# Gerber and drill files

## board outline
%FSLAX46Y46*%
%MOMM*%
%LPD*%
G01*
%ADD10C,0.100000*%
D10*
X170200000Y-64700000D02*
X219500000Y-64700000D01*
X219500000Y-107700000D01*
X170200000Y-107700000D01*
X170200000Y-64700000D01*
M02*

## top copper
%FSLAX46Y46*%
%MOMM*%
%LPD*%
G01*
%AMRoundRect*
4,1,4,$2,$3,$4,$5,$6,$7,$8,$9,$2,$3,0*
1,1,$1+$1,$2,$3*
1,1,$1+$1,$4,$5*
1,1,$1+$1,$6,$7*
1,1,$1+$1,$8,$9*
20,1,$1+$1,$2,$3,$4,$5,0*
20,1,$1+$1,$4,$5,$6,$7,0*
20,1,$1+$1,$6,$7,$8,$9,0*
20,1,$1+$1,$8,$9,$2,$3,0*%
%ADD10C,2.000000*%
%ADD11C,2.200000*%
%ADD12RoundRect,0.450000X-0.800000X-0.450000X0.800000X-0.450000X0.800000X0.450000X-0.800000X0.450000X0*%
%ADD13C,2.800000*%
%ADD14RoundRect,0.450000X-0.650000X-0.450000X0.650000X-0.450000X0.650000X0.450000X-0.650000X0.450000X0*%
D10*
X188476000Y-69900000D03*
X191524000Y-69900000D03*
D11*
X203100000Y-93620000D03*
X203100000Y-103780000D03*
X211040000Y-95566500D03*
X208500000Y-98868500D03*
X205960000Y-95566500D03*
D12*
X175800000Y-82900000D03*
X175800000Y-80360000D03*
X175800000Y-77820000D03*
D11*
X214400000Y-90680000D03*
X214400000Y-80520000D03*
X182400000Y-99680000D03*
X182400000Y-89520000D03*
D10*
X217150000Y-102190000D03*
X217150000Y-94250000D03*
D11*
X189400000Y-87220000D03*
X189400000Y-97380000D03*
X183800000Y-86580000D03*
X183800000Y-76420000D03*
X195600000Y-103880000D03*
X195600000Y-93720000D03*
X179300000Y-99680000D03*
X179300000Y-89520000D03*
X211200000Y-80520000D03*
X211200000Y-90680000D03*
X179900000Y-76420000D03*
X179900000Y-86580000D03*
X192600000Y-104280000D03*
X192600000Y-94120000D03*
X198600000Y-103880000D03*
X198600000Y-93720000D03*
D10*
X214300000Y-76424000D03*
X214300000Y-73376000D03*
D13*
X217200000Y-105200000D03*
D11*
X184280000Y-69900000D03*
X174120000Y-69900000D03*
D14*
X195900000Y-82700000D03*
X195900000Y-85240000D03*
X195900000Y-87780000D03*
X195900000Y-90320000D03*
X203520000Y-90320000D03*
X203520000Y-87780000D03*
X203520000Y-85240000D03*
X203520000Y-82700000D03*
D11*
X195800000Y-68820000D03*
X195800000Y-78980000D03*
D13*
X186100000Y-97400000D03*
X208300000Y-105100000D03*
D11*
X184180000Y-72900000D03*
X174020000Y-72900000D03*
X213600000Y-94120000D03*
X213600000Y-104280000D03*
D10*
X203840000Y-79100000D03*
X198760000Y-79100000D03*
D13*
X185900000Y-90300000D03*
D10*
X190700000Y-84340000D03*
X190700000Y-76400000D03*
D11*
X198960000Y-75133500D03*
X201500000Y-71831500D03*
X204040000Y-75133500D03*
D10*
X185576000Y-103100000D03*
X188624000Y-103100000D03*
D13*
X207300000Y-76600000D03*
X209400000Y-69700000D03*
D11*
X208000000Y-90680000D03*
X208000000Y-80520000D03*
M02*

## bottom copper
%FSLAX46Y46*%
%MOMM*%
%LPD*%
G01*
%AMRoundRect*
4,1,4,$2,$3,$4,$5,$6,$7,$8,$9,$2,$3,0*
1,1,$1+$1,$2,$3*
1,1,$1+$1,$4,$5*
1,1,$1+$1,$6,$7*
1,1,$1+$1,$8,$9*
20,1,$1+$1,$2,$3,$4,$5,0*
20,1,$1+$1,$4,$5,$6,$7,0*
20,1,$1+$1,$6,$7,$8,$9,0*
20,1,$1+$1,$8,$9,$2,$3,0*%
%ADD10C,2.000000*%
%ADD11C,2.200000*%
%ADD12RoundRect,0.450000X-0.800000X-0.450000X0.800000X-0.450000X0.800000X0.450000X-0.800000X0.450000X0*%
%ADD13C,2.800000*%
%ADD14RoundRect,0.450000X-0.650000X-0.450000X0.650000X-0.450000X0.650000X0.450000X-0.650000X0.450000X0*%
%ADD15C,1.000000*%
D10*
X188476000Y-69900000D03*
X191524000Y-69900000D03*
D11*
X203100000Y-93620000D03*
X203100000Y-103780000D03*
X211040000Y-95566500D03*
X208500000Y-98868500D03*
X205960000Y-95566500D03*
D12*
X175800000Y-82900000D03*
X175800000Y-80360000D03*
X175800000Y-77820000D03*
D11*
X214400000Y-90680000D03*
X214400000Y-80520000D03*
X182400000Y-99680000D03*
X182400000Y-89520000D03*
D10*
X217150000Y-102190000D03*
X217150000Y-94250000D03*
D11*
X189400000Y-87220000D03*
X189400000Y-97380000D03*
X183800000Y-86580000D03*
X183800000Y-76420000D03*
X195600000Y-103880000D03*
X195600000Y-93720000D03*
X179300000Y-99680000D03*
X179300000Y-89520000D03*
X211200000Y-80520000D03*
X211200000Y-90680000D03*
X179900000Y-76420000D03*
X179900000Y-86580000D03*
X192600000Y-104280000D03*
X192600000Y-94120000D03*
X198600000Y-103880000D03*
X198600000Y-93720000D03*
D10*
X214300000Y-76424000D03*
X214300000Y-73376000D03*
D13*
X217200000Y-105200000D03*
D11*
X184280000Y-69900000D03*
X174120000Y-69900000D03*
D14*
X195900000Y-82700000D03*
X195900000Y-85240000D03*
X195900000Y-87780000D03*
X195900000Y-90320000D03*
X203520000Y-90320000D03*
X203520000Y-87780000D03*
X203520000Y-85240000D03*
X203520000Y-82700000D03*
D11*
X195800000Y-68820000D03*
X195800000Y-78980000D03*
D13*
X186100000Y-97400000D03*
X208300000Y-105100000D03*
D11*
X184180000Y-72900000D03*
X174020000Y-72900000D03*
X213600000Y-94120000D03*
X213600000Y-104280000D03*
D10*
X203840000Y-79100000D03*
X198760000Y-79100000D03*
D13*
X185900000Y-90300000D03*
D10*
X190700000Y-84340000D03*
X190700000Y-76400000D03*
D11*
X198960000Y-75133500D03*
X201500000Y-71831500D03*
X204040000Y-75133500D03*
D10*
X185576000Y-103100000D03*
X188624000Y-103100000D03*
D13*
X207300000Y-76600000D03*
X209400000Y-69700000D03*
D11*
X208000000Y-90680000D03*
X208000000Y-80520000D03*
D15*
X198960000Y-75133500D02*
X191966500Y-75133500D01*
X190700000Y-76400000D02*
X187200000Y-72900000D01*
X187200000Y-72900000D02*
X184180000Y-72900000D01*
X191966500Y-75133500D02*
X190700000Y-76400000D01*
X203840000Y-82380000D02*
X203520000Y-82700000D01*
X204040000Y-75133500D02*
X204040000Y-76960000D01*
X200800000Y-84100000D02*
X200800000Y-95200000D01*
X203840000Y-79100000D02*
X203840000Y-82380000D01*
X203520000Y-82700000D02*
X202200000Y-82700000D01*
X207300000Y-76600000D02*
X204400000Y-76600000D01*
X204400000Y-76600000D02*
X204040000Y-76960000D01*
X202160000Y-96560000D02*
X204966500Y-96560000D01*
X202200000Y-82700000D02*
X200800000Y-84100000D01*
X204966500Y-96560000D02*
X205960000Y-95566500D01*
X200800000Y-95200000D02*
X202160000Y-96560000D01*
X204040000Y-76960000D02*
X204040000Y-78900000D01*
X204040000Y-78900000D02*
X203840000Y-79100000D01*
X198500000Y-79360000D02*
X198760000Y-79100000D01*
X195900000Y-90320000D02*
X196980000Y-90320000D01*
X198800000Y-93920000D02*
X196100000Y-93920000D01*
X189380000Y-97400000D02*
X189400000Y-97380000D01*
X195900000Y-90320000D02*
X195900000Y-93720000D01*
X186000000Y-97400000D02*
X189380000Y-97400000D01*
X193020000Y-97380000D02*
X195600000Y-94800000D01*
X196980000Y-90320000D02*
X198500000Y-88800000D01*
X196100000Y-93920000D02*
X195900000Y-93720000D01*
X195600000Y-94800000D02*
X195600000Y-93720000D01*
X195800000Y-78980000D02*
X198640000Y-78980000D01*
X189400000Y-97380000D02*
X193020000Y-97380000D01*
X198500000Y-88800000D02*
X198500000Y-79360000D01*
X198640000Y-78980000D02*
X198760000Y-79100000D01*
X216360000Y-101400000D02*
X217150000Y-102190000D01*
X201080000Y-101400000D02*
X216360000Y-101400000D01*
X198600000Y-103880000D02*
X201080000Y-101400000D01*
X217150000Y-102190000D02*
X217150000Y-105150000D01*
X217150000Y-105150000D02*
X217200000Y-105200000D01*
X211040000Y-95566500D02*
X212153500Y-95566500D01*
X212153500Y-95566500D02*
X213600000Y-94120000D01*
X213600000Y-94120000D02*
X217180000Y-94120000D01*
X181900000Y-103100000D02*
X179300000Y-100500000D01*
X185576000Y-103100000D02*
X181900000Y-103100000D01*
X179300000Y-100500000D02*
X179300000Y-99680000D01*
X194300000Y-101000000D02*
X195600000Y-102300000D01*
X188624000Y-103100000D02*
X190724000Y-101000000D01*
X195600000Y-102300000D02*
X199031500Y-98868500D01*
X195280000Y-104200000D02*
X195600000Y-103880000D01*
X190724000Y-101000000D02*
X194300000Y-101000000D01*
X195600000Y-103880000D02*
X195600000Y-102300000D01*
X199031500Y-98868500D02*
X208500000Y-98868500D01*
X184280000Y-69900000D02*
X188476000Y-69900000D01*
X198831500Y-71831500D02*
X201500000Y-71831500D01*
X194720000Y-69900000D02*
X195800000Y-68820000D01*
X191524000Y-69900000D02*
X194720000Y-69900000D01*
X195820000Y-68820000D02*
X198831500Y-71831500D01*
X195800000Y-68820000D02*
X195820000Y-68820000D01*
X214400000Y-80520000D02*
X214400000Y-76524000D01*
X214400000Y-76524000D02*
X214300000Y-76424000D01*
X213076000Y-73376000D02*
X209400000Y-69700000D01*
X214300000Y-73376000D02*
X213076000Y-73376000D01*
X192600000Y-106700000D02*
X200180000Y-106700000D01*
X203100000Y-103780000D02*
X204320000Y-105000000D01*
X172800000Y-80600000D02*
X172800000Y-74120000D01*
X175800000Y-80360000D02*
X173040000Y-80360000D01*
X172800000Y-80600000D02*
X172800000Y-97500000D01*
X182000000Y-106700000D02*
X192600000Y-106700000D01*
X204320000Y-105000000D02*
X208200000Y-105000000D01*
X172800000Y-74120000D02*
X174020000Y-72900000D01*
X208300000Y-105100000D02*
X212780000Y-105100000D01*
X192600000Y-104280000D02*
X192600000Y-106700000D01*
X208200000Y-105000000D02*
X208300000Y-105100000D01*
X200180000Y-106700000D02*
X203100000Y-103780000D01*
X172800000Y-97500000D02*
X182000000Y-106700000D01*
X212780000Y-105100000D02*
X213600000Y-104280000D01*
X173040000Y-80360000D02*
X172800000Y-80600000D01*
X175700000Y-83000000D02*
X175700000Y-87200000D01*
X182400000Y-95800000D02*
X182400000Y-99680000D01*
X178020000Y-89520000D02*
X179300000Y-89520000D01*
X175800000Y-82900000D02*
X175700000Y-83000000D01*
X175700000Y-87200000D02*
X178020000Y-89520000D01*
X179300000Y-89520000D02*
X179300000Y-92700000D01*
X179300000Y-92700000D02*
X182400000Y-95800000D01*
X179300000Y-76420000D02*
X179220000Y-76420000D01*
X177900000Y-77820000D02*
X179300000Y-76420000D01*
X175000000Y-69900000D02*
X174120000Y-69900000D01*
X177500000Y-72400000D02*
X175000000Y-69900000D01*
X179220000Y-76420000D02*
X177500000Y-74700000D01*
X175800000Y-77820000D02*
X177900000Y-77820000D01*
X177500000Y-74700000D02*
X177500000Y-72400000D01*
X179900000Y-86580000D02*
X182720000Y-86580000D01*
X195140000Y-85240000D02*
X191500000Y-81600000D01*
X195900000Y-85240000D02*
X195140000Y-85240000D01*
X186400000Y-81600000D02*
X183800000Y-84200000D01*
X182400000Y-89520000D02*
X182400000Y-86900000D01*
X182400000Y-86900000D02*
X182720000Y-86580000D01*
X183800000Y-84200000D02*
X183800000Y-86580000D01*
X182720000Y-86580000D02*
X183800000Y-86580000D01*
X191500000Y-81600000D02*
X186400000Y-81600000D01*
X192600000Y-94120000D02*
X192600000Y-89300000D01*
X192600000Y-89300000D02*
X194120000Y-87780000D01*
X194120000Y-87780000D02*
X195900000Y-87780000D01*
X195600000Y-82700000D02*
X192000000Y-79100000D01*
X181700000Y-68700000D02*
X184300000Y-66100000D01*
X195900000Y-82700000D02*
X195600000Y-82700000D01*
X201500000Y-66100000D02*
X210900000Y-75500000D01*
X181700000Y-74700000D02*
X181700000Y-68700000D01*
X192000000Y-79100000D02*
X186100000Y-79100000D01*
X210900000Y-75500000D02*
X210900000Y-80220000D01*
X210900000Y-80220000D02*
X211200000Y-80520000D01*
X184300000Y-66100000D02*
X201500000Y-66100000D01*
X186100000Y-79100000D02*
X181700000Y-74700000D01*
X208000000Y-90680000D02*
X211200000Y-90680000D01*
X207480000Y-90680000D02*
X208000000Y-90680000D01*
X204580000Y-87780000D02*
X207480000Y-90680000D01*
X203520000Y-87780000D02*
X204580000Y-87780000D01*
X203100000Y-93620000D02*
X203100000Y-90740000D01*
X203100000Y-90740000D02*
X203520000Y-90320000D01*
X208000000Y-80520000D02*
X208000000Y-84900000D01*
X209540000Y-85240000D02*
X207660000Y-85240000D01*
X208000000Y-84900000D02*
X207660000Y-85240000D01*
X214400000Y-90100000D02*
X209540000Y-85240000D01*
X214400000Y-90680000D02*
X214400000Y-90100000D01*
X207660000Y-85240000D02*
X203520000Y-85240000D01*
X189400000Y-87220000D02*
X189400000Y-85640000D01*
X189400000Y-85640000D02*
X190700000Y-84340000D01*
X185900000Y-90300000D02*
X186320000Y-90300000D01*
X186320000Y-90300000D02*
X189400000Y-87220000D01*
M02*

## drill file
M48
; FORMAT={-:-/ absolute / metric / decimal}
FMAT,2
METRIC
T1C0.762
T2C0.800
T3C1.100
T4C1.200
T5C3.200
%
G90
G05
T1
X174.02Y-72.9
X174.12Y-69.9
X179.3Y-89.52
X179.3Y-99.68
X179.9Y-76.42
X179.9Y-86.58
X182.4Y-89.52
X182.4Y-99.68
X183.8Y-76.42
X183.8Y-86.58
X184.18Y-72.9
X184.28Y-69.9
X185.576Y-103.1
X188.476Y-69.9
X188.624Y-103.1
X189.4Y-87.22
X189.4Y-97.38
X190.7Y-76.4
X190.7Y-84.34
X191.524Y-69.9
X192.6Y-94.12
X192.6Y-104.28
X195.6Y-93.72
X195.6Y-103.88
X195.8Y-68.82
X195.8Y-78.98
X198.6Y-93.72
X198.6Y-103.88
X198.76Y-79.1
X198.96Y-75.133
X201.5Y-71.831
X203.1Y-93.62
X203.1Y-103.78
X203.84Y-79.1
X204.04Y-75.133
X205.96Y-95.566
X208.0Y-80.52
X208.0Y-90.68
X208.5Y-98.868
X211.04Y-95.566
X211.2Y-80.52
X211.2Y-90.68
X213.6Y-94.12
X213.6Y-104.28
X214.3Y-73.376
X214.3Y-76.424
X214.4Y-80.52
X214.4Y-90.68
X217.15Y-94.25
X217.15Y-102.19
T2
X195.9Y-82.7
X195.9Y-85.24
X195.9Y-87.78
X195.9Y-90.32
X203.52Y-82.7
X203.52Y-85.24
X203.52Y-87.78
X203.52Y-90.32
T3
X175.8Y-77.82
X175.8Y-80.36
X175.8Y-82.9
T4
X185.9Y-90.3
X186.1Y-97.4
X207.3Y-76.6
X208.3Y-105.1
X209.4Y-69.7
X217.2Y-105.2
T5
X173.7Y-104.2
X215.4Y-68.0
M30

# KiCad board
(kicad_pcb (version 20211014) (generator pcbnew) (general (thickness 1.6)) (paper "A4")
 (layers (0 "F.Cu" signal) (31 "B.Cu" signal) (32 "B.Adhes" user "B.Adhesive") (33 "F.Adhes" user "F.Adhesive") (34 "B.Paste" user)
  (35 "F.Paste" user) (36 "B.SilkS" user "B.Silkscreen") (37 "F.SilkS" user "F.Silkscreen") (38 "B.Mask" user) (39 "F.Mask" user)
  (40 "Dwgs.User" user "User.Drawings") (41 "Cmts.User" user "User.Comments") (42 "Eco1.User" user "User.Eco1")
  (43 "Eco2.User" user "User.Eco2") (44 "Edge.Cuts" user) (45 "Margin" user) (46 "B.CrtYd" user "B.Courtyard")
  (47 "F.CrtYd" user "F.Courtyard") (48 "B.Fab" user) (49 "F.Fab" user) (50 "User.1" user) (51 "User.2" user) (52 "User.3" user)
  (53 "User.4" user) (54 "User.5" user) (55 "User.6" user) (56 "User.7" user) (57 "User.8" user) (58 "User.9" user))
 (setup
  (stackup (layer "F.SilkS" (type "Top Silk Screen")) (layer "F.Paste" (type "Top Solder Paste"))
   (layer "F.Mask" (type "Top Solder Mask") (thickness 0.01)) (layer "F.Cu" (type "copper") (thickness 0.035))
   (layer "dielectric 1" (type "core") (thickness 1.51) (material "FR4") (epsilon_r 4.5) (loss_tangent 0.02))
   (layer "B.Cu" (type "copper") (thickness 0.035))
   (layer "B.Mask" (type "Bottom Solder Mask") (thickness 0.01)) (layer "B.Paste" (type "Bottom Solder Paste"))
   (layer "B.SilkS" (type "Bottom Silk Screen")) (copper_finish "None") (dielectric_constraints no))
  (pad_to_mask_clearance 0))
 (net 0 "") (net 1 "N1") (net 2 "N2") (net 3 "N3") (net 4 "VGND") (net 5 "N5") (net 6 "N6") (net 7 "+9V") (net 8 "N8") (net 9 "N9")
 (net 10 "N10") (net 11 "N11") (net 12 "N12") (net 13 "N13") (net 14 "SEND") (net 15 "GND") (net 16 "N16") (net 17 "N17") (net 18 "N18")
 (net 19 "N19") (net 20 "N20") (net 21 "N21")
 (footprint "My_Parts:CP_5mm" (layer "F.Cu") (at 190 69.9)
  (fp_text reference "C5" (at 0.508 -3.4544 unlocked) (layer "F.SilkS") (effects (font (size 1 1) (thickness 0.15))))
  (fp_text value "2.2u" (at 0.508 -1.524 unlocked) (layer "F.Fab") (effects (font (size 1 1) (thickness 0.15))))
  (pad "1" thru_hole circle (at -1.524 0) (size 2 2) (drill 0.762) (layers *.Cu *.Mask) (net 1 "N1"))
  (pad "2" thru_hole circle (at 1.524 0) (size 2 2) (drill 0.762) (layers *.Cu *.Mask) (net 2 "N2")))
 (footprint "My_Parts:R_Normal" (layer "F.Cu") (at 203.1 98.7 -90)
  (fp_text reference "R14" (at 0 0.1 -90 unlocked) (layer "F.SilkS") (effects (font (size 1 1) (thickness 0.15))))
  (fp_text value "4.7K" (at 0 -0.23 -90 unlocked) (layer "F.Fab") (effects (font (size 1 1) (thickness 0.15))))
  (pad "1" thru_hole circle (at -5.08 0 270) (size 2.2 2.2) (drill 0.762) (layers *.Cu *.Mask) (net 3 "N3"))
  (pad "2" thru_hole circle (at 5.08 0 270) (size 2.2 2.2) (drill 0.762) (layers *.Cu *.Mask) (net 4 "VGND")))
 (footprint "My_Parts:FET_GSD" (layer "F.Cu") (at 211.04 96.5825 180)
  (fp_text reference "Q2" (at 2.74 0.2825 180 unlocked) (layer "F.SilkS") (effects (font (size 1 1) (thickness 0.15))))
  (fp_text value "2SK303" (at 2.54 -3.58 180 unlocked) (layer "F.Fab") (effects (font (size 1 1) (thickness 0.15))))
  (pad "1" thru_hole circle (at 0 1.016 180) (size 2.2 2.2) (drill 0.762) (layers *.Cu *.Mask) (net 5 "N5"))
  (pad "2" thru_hole circle (at 2.54 -2.286 180) (size 2.2 2.2) (drill 0.762) (layers *.Cu *.Mask) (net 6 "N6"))
  (pad "3" thru_hole circle (at 5.08 1.016 180) (size 2.2 2.2) (drill 0.762) (layers *.Cu *.Mask) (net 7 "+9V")))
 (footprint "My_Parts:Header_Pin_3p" (layer "F.Cu") (at 175.8 82.9)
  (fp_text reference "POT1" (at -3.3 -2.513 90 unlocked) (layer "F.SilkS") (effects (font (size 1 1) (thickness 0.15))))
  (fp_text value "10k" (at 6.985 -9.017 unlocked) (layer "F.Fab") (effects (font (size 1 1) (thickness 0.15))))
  (pad "1" thru_hole roundrect (at 0 0) (size 2.5 1.8) (drill 1.1) (layers *.Cu *.Mask) (roundrect_rratio 0.25) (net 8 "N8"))
  (pad "2" thru_hole roundrect (at 0 -2.54) (size 2.5 1.8) (drill 1.1) (layers *.Cu *.Mask) (roundrect_rratio 0.25) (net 4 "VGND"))
  (pad "3" thru_hole roundrect (at 0 -5.08) (size 2.5 1.8) (drill 1.1) (layers *.Cu *.Mask) (roundrect_rratio 0.25) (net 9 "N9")))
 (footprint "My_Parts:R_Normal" (layer "F.Cu") (at 214.4 85.6 90)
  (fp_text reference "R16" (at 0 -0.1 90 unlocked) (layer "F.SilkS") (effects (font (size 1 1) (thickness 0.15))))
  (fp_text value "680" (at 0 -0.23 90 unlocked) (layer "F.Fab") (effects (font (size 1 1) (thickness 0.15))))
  (pad "1" thru_hole circle (at -5.08 0 90) (size 2.2 2.2) (drill 0.762) (layers *.Cu *.Mask) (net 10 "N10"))
  (pad "2" thru_hole circle (at 5.08 0 90) (size 2.2 2.2) (drill 0.762) (layers *.Cu *.Mask) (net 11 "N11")))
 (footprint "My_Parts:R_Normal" (layer "F.Cu") (at 182.4 94.6 90)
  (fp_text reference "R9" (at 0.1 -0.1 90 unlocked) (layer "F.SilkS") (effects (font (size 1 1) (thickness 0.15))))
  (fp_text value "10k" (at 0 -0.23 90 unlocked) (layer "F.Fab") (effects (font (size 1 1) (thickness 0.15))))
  (pad "1" thru_hole circle (at -5.08 0 90) (size 2.2 2.2) (drill 0.762) (layers *.Cu *.Mask) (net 8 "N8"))
  (pad "2" thru_hole circle (at 5.08 0 90) (size 2.2 2.2) (drill 0.762) (layers *.Cu *.Mask) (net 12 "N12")))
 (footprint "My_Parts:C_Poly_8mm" (layer "F.Cu") (at 217.15 99.65 90)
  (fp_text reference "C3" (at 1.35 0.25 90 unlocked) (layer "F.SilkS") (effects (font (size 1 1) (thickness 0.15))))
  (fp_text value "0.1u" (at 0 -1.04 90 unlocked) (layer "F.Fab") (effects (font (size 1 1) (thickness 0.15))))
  (pad "1" thru_hole circle (at -2.54 0 90) (size 2 2) (drill 0.762) (layers *.Cu *.Mask) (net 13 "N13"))
  (pad "2" thru_hole circle (at 5.4 0 90) (size 2 2) (drill 0.762) (layers *.Cu *.Mask) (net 5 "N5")))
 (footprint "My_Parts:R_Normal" (layer "F.Cu") (at 189.4 92.3 -90)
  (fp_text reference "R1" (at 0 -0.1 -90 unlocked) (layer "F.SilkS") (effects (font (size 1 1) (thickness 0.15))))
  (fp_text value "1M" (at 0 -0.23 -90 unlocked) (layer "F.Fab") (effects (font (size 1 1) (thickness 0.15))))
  (pad "1" thru_hole circle (at -5.08 0 270) (size 2.2 2.2) (drill 0.762) (layers *.Cu *.Mask) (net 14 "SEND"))
  (pad "2" thru_hole circle (at 5.08 0 270) (size 2.2 2.2) (drill 0.762) (layers *.Cu *.Mask) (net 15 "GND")))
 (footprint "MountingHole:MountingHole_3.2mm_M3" (layer "F.Cu") (at 173.7 104.2)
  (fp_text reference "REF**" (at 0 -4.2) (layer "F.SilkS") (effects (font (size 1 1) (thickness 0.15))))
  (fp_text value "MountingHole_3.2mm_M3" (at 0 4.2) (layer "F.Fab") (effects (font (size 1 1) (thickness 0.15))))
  (pad "" np_thru_hole circle (at 0 0) (size 3.2 3.2) (drill 3.2) (layers F&B.Cu *.Mask)))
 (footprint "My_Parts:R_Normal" (layer "F.Cu") (at 183.8 81.5 90)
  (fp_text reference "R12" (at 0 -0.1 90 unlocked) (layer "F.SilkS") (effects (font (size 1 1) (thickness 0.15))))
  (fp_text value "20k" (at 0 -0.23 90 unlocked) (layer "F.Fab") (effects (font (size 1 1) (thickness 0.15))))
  (pad "1" thru_hole circle (at -5.08 0 90) (size 2.2 2.2) (drill 0.762) (layers *.Cu *.Mask) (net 12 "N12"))
  (pad "2" thru_hole circle (at 5.08 0 90) (size 2.2 2.2) (drill 0.762) (layers *.Cu *.Mask) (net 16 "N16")))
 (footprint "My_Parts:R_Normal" (layer "F.Cu") (at 195.6 98.8 90)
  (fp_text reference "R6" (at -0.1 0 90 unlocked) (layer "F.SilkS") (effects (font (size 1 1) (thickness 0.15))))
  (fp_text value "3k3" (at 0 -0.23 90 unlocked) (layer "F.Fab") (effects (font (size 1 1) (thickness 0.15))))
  (pad "1" thru_hole circle (at -5.08 0 90) (size 2.2 2.2) (drill 0.762) (layers *.Cu *.Mask) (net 6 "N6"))
  (pad "2" thru_hole circle (at 5.08 0 90) (size 2.2 2.2) (drill 0.762) (layers *.Cu *.Mask) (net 15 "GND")))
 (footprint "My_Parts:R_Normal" (layer "F.Cu") (at 179.3 94.6 90)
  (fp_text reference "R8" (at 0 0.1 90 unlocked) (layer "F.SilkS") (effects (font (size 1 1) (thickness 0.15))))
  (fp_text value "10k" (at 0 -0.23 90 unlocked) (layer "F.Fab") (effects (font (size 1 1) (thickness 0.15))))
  (pad "1" thru_hole circle (at -5.08 0 90) (size 2.2 2.2) (drill 0.762) (layers *.Cu *.Mask) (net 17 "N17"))
  (pad "2" thru_hole circle (at 5.08 0 90) (size 2.2 2.2) (drill 0.762) (layers *.Cu *.Mask) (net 8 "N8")))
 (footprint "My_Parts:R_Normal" (layer "F.Cu") (at 211.2 85.6 -90)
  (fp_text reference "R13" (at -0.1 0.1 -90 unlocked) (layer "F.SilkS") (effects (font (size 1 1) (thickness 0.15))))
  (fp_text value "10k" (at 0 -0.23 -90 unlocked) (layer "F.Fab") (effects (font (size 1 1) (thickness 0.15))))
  (pad "1" thru_hole circle (at -5.08 0 270) (size 2.2 2.2) (drill 0.762) (layers *.Cu *.Mask) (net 16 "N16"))
  (pad "2" thru_hole circle (at 5.08 0 270) (size 2.2 2.2) (drill 0.762) (layers *.Cu *.Mask) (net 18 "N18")))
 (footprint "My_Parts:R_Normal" (layer "F.Cu") (at 179.9 81.5 -90)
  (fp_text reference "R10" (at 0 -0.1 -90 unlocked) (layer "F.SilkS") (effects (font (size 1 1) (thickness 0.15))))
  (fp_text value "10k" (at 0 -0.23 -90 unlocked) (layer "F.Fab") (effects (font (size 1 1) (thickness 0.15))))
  (pad "1" thru_hole circle (at -5.08 0 270) (size 2.2 2.2) (drill 0.762) (layers *.Cu *.Mask) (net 9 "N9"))
  (pad "2" thru_hole circle (at 5.08 0 270) (size 2.2 2.2) (drill 0.762) (layers *.Cu *.Mask) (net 12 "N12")))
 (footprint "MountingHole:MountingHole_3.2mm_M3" (layer "F.Cu") (at 215.4 68)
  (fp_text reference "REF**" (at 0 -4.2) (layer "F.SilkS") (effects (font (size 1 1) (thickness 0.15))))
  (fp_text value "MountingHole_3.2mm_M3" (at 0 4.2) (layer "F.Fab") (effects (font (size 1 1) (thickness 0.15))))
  (pad "" np_thru_hole circle (at 0 0) (size 3.2 3.2) (drill 3.2) (layers *.Cu *.Mask)))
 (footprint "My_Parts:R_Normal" (layer "F.Cu") (at 192.6 99.2 90)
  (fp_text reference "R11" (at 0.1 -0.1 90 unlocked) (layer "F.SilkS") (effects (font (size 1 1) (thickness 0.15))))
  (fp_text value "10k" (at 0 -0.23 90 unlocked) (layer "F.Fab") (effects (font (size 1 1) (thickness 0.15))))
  (pad "1" thru_hole circle (at -5.08 0 90) (size 2.2 2.2) (drill 0.762) (layers *.Cu *.Mask) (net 4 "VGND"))
  (pad "2" thru_hole circle (at 5.08 0 90) (size 2.2 2.2) (drill 0.762) (layers *.Cu *.Mask) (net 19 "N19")))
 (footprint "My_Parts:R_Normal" (layer "F.Cu") (at 198.6 98.8 90)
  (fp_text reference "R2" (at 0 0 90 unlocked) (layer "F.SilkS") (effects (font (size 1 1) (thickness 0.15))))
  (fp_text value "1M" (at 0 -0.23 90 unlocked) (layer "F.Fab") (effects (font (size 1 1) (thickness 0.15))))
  (pad "1" thru_hole circle (at -5.08 0 90) (size 2.2 2.2) (drill 0.762) (layers *.Cu *.Mask) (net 13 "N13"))
  (pad "2" thru_hole circle (at 5.08 0 90) (size 2.2 2.2) (drill 0.762) (layers *.Cu *.Mask) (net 15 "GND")))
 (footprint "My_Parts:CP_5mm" (layer "F.Cu") (at 214.3 74.9 90)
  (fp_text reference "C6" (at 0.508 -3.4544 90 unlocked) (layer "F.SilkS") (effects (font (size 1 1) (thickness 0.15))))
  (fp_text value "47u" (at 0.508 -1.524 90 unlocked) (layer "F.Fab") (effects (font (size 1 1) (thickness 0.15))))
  (pad "1" thru_hole circle (at -1.524 0 90) (size 2 2) (drill 0.762) (layers *.Cu *.Mask) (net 11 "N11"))
  (pad "2" thru_hole circle (at 1.524 0 90) (size 2 2) (drill 0.762) (layers *.Cu *.Mask) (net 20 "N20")))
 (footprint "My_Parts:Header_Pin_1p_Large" (layer "F.Cu") (at 217.2 105.2)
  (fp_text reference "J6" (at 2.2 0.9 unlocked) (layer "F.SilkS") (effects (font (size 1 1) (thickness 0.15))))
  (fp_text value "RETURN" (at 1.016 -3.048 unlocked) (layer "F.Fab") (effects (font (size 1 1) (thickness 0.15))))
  (pad "1" thru_hole circle (at 0 0) (size 2.8 2.8) (drill 1.2) (layers *.Cu *.Mask) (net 13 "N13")))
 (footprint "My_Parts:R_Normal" (layer "F.Cu") (at 179.2 69.9 180)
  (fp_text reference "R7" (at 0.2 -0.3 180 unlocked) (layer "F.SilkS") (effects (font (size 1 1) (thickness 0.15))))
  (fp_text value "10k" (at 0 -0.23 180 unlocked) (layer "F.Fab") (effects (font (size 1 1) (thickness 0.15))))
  (pad "1" thru_hole circle (at -5.08 0 180) (size 2.2 2.2) (drill 0.762) (layers *.Cu *.Mask) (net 1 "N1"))
  (pad "2" thru_hole circle (at 5.08 0 180) (size 2.2 2.2) (drill 0.762) (layers *.Cu *.Mask) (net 9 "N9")))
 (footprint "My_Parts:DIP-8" (layer "F.Cu") (at 197.17 83.2)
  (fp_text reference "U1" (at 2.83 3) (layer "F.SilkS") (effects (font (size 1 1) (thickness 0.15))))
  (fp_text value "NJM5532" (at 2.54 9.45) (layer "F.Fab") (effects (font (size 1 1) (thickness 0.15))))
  (pad "1" thru_hole roundrect (at -1.27 -0.5) (size 2.2 1.8) (drill 0.8) (layers *.Cu *.Mask) (roundrect_rratio 0.25) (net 16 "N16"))
  (pad "2" thru_hole roundrect (at -1.27 2.04) (size 2.2 1.8) (drill 0.8) (layers *.Cu *.Mask) (roundrect_rratio 0.25) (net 12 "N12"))
  (pad "3" thru_hole roundrect (at -1.27 4.58) (size 2.2 1.8) (drill 0.8) (layers *.Cu *.Mask) (roundrect_rratio 0.25) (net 19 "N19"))
  (pad "4" thru_hole roundrect (at -1.27 7.12) (size 2.2 1.8) (drill 0.8) (layers *.Cu *.Mask) (roundrect_rratio 0.25) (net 15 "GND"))
  (pad "5" thru_hole roundrect (at 6.35 7.12) (size 2.2 1.8) (drill 0.8) (layers *.Cu *.Mask) (roundrect_rratio 0.25) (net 3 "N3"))
  (pad "6" thru_hole roundrect (at 6.35 4.58) (size 2.2 1.8) (drill 0.8) (layers *.Cu *.Mask) (roundrect_rratio 0.25) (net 18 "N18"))
  (pad "7" thru_hole roundrect (at 6.35 2.04) (size 2.2 1.8) (drill 0.8) (layers *.Cu *.Mask) (roundrect_rratio 0.25) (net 10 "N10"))
  (pad "8" thru_hole roundrect (at 6.35 -0.5) (size 2.2 1.8) (drill 0.8) (layers *.Cu *.Mask) (roundrect_rratio 0.25) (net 7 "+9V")))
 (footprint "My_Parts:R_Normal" (layer "F.Cu") (at 195.8 73.9 -90)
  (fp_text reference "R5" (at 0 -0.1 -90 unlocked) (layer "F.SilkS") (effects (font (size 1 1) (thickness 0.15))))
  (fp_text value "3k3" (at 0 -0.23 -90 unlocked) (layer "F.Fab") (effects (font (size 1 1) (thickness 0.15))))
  (pad "1" thru_hole circle (at -5.08 0 270) (size 2.2 2.2) (drill 0.762) (layers *.Cu *.Mask) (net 2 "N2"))
  (pad "2" thru_hole circle (at 5.08 0 270) (size 2.2 2.2) (drill 0.762) (layers *.Cu *.Mask) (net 15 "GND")))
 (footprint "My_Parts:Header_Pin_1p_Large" (layer "F.Cu") (at 186.1 97.4)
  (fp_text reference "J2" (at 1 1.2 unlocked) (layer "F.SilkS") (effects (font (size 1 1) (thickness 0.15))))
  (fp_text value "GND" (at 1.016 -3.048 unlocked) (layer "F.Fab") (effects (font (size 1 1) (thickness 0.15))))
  (pad "1" thru_hole circle (at 0 0) (size 2.8 2.8) (drill 1.2) (layers *.Cu *.Mask) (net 15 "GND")))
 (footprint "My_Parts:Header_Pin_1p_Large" (layer "F.Cu") (at 208.3 105.1)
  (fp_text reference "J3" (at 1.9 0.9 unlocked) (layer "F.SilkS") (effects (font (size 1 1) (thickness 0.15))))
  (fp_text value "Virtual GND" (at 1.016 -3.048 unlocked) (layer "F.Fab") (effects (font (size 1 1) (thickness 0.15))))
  (pad "1" thru_hole circle (at 0 0) (size 2.8 2.8) (drill 1.2) (layers *.Cu *.Mask) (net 4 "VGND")))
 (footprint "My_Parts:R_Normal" (layer "F.Cu") (at 179.1 72.9 180)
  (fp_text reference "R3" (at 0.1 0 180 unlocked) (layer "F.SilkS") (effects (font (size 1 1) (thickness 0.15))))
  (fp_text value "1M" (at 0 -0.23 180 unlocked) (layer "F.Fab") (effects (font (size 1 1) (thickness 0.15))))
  (pad "1" thru_hole circle (at -5.08 0 180) (size 2.2 2.2) (drill 0.762) (layers *.Cu *.Mask) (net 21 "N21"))
  (pad "2" thru_hole circle (at 5.08 0 180) (size 2.2 2.2) (drill 0.762) (layers *.Cu *.Mask) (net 4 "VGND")))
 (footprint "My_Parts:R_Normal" (layer "F.Cu") (at 213.6 99.2 -90)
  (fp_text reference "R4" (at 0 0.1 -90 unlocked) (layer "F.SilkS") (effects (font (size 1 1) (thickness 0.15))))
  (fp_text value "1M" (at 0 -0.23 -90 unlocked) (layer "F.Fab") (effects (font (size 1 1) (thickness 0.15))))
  (pad "1" thru_hole circle (at -5.08 0 270) (size 2.2 2.2) (drill 0.762) (layers *.Cu *.Mask) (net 5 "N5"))
  (pad "2" thru_hole circle (at 5.08 0 270) (size 2.2 2.2) (drill 0.762) (layers *.Cu *.Mask) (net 4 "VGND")))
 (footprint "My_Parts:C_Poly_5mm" (layer "F.Cu") (at 201.3 79.1 180)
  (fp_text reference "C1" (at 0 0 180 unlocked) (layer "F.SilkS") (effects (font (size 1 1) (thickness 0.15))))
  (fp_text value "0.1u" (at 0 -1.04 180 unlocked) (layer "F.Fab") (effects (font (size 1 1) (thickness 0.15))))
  (pad "1" thru_hole circle (at -2.54 0 180) (size 2 2) (drill 0.762) (layers *.Cu *.Mask) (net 7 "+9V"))
  (pad "2" thru_hole circle (at 2.54 0 180) (size 2 2) (drill 0.762) (layers *.Cu *.Mask) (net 15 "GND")))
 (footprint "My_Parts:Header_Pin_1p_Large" (layer "F.Cu") (at 185.9 90.3)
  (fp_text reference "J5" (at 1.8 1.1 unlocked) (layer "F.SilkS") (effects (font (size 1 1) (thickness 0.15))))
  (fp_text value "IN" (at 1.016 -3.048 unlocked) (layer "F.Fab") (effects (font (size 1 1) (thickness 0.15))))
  (pad "1" thru_hole circle (at 0 0) (size 2.8 2.8) (drill 1.2) (layers *.Cu *.Mask) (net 14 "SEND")))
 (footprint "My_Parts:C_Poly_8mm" (layer "F.Cu") (at 190.7 81.8 90)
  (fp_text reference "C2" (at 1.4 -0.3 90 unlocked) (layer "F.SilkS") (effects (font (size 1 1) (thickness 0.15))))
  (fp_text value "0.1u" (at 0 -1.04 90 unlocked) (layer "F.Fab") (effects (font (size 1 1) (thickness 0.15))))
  (pad "1" thru_hole circle (at -2.54 0 90) (size 2 2) (drill 0.762) (layers *.Cu *.Mask) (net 14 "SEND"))
  (pad "2" thru_hole circle (at 5.4 0 90) (size 2 2) (drill 0.762) (layers *.Cu *.Mask) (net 21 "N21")))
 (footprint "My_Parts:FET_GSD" (layer "F.Cu") (at 198.96 74.1175)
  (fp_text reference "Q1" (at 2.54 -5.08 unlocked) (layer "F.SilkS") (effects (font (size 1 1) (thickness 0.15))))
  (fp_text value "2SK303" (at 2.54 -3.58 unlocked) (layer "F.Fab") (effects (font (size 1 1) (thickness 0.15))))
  (pad "1" thru_hole circle (at 0 1.016) (size 2.2 2.2) (drill 0.762) (layers *.Cu *.Mask) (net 21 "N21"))
  (pad "2" thru_hole circle (at 2.54 -2.286) (size 2.2 2.2) (drill 0.762) (layers *.Cu *.Mask) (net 2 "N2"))
  (pad "3" thru_hole circle (at 5.08 1.016) (size 2.2 2.2) (drill 0.762) (layers *.Cu *.Mask) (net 7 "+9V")))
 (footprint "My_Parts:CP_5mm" (layer "F.Cu") (at 187.1 103.1)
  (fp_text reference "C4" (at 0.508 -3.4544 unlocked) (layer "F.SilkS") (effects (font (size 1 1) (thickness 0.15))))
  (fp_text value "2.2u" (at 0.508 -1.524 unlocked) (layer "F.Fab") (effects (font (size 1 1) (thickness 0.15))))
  (pad "1" thru_hole circle (at -1.524 0) (size 2 2) (drill 0.762) (layers *.Cu *.Mask) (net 17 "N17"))
  (pad "2" thru_hole circle (at 1.524 0) (size 2 2) (drill 0.762) (layers *.Cu *.Mask) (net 6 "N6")))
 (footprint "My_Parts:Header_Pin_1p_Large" (layer "F.Cu") (at 207.3 76.6)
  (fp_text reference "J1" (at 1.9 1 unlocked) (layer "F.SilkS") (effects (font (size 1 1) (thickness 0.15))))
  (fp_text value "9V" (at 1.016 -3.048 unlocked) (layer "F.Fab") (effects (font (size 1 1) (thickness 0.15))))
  (pad "1" thru_hole circle (at 0 0) (size 2.8 2.8) (drill 1.2) (layers *.Cu *.Mask) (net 7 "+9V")))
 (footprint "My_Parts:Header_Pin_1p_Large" (layer "F.Cu") (at 209.4 69.7)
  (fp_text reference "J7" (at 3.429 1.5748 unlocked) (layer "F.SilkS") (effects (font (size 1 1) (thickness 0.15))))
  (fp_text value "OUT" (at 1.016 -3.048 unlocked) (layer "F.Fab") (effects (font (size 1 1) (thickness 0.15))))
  (pad "1" thru_hole circle (at 0 0) (size 2.8 2.8) (drill 1.2) (layers *.Cu *.Mask) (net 20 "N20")))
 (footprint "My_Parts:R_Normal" (layer "F.Cu") (at 208 85.6 90)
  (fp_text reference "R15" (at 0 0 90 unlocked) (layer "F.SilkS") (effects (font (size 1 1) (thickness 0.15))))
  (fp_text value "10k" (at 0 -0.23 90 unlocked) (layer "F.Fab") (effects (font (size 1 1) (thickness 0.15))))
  (pad "1" thru_hole circle (at -5.08 0 90) (size 2.2 2.2) (drill 0.762) (layers *.Cu *.Mask) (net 18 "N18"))
  (pad "2" thru_hole circle (at 5.08 0 90) (size 2.2 2.2) (drill 0.762) (layers *.Cu *.Mask) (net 10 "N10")))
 (gr_rect (start 170.2 64.7) (end 219.5 107.7) (layer "Edge.Cuts") (width 0.1) (fill none))
 (segment (start 198.96 75.1335) (end 191.9665 75.1335) (width 1) (layer "B.Cu") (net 21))
 (segment (start 190.7 76.4) (end 187.2 72.9) (width 1) (layer "B.Cu") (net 21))
 (segment (start 187.2 72.9) (end 184.18 72.9) (width 1) (layer "B.Cu") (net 21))
 (segment (start 191.9665 75.1335) (end 190.7 76.4) (width 1) (layer "B.Cu") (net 21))
 (segment (start 203.84 82.38) (end 203.52 82.7) (width 1) (layer "B.Cu") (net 7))
 (segment (start 204.04 75.1335) (end 204.04 76.96) (width 1) (layer "B.Cu") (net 7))
 (segment (start 200.8 84.1) (end 200.8 95.2) (width 1) (layer "B.Cu") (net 7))
 (segment (start 203.84 79.1) (end 203.84 82.38) (width 1) (layer "B.Cu") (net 7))
 (segment (start 203.52 82.7) (end 202.2 82.7) (width 1) (layer "B.Cu") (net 7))
 (segment (start 207.3 76.6) (end 204.4 76.6) (width 1) (layer "B.Cu") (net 7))
 (segment (start 204.4 76.6) (end 204.04 76.96) (width 1) (layer "B.Cu") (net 7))
 (segment (start 202.16 96.56) (end 204.9665 96.56) (width 1) (layer "B.Cu") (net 7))
 (segment (start 202.2 82.7) (end 200.8 84.1) (width 1) (layer "B.Cu") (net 7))
 (segment (start 204.9665 96.56) (end 205.96 95.5665) (width 1) (layer "B.Cu") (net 7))
 (segment (start 200.8 95.2) (end 202.16 96.56) (width 1) (layer "B.Cu") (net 7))
 (segment (start 204.04 76.96) (end 204.04 78.9) (width 1) (layer "B.Cu") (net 7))
 (segment (start 204.04 78.9) (end 203.84 79.1) (width 1) (layer "B.Cu") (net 7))
 (segment (start 198.5 79.36) (end 198.76 79.1) (width 1) (layer "B.Cu") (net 15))
 (segment (start 195.9 90.32) (end 196.98 90.32) (width 1) (layer "B.Cu") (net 15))
 (segment (start 198.8 93.92) (end 196.1 93.92) (width 1) (layer "B.Cu") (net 15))
 (segment (start 189.38 97.4) (end 189.4 97.38) (width 1) (layer "B.Cu") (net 15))
 (segment (start 195.9 90.32) (end 195.9 93.72) (width 1) (layer "B.Cu") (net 15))
 (segment (start 186 97.4) (end 189.38 97.4) (width 1) (layer "B.Cu") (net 15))
 (segment (start 193.02 97.38) (end 195.6 94.8) (width 1) (layer "B.Cu") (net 15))
 (segment (start 196.98 90.32) (end 198.5 88.8) (width 1) (layer "B.Cu") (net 15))
 (segment (start 196.1 93.92) (end 195.9 93.72) (width 1) (layer "B.Cu") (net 15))
 (segment (start 195.6 94.8) (end 195.6 93.72) (width 1) (layer "B.Cu") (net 15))
 (segment (start 195.8 78.98) (end 198.64 78.98) (width 1) (layer "B.Cu") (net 15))
 (segment (start 189.4 97.38) (end 193.02 97.38) (width 1) (layer "B.Cu") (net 15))
 (segment (start 198.5 88.8) (end 198.5 79.36) (width 1) (layer "B.Cu") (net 15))
 (segment (start 198.64 78.98) (end 198.76 79.1) (width 1) (layer "B.Cu") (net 15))
 (segment (start 216.36 101.4) (end 217.15 102.19) (width 1) (layer "B.Cu") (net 13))
 (segment (start 201.08 101.4) (end 216.36 101.4) (width 1) (layer "B.Cu") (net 13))
 (segment (start 198.6 103.88) (end 201.08 101.4) (width 1) (layer "B.Cu") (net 13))
 (segment (start 217.15 102.19) (end 217.15 105.15) (width 1) (layer "B.Cu") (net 13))
 (segment (start 217.15 105.15) (end 217.2 105.2) (width 1) (layer "B.Cu") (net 13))
 (segment (start 211.04 95.5665) (end 212.1535 95.5665) (width 1) (layer "B.Cu") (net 5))
 (segment (start 212.1535 95.5665) (end 213.6 94.12) (width 1) (layer "B.Cu") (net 5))
 (segment (start 213.6 94.12) (end 217.18 94.12) (width 1) (layer "B.Cu") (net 5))
 (segment (start 181.9 103.1) (end 179.3 100.5) (width 1) (layer "B.Cu") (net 17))
 (segment (start 185.576 103.1) (end 181.9 103.1) (width 1) (layer "B.Cu") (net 17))
 (segment (start 179.3 100.5) (end 179.3 99.68) (width 1) (layer "B.Cu") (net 17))
 (segment (start 194.3 101) (end 195.6 102.3) (width 1) (layer "B.Cu") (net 6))
 (segment (start 188.624 103.1) (end 190.724 101) (width 1) (layer "B.Cu") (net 6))
 (segment (start 195.6 102.3) (end 199.0315 98.8685) (width 1) (layer "B.Cu") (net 6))
 (segment (start 195.28 104.2) (end 195.6 103.88) (width 1) (layer "B.Cu") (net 6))
 (segment (start 190.724 101) (end 194.3 101) (width 1) (layer "B.Cu") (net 6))
 (segment (start 195.6 103.88) (end 195.6 102.3) (width 1) (layer "B.Cu") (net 6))
 (segment (start 199.0315 98.8685) (end 208.5 98.8685) (width 1) (layer "B.Cu") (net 6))
 (segment (start 184.28 69.9) (end 188.476 69.9) (width 1) (layer "B.Cu") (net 1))
 (segment (start 198.8315 71.8315) (end 201.5 71.8315) (width 1) (layer "B.Cu") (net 2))
 (segment (start 194.72 69.9) (end 195.8 68.82) (width 1) (layer "B.Cu") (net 2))
 (segment (start 191.524 69.9) (end 194.72 69.9) (width 1) (layer "B.Cu") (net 2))
 (segment (start 195.82 68.82) (end 198.8315 71.8315) (width 1) (layer "B.Cu") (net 2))
 (segment (start 195.8 68.82) (end 195.82 68.82) (width 1) (layer "B.Cu") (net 2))
 (segment (start 214.4 80.52) (end 214.4 76.524) (width 1) (layer "B.Cu") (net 11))
 (segment (start 214.4 76.524) (end 214.3 76.424) (width 1) (layer "B.Cu") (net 11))
 (segment (start 213.076 73.376) (end 209.4 69.7) (width 1) (layer "B.Cu") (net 20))
 (segment (start 214.3 73.376) (end 213.076 73.376) (width 1) (layer "B.Cu") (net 20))
 (segment (start 192.6 106.7) (end 200.18 106.7) (width 1) (layer "B.Cu") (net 4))
 (segment (start 203.1 103.78) (end 204.32 105) (width 1) (layer "B.Cu") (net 4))
 (segment (start 172.8 80.6) (end 172.8 74.12) (width 1) (layer "B.Cu") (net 4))
 (segment (start 175.8 80.36) (end 173.04 80.36) (width 1) (layer "B.Cu") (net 4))
 (segment (start 172.8 80.6) (end 172.8 97.5) (width 1) (layer "B.Cu") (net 4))
 (segment (start 182 106.7) (end 192.6 106.7) (width 1) (layer "B.Cu") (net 4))
 (segment (start 204.32 105) (end 208.2 105) (width 1) (layer "B.Cu") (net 4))
 (segment (start 172.8 74.12) (end 174.02 72.9) (width 1) (layer "B.Cu") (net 4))
 (segment (start 208.3 105.1) (end 212.78 105.1) (width 1) (layer "B.Cu") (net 4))
 (segment (start 192.6 104.28) (end 192.6 106.7) (width 1) (layer "B.Cu") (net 4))
 (segment (start 208.2 105) (end 208.3 105.1) (width 1) (layer "B.Cu") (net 4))
 (segment (start 200.18 106.7) (end 203.1 103.78) (width 1) (layer "B.Cu") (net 4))
 (segment (start 172.8 97.5) (end 182 106.7) (width 1) (layer "B.Cu") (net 4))
 (segment (start 212.78 105.1) (end 213.6 104.28) (width 1) (layer "B.Cu") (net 4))
 (segment (start 173.04 80.36) (end 172.8 80.6) (width 1) (layer "B.Cu") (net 4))
 (segment (start 175.7 83) (end 175.7 87.2) (width 1) (layer "B.Cu") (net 8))
 (segment (start 182.4 95.8) (end 182.4 99.68) (width 1) (layer "B.Cu") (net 8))
 (segment (start 178.02 89.52) (end 179.3 89.52) (width 1) (layer "B.Cu") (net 8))
 (segment (start 175.8 82.9) (end 175.7 83) (width 1) (layer "B.Cu") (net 8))
 (segment (start 175.7 87.2) (end 178.02 89.52) (width 1) (layer "B.Cu") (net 8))
 (segment (start 179.3 89.52) (end 179.3 92.7) (width 1) (layer "B.Cu") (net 8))
 (segment (start 179.3 92.7) (end 182.4 95.8) (width 1) (layer "B.Cu") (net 8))
 (segment (start 179.3 76.42) (end 179.22 76.42) (width 1) (layer "B.Cu") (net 9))
 (segment (start 177.9 77.82) (end 179.3 76.42) (width 1) (layer "B.Cu") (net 9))
 (segment (start 175 69.9) (end 174.12 69.9) (width 1) (layer "B.Cu") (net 9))
 (segment (start 177.5 72.4) (end 175 69.9) (width 1) (layer "B.Cu") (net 9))
 (segment (start 179.22 76.42) (end 177.5 74.7) (width 1) (layer "B.Cu") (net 9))
 (segment (start 175.8 77.82) (end 177.9 77.82) (width 1) (layer "B.Cu") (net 9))
 (segment (start 177.5 74.7) (end 177.5 72.4) (width 1) (layer "B.Cu") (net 9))
 (segment (start 179.9 86.58) (end 182.72 86.58) (width 1) (layer "B.Cu") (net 12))
 (segment (start 195.14 85.24) (end 191.5 81.6) (width 1) (layer "B.Cu") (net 12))
 (segment (start 195.9 85.24) (end 195.14 85.24) (width 1) (layer "B.Cu") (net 12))
 (segment (start 186.4 81.6) (end 183.8 84.2) (width 1) (layer "B.Cu") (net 12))
 (segment (start 182.4 89.52) (end 182.4 86.9) (width 1) (layer "B.Cu") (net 12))
 (segment (start 182.4 86.9) (end 182.72 86.58) (width 1) (layer "B.Cu") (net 12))
 (segment (start 183.8 84.2) (end 183.8 86.58) (width 1) (layer "B.Cu") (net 12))
 (segment (start 182.72 86.58) (end 183.8 86.58) (width 1) (layer "B.Cu") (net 12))
 (segment (start 191.5 81.6) (end 186.4 81.6) (width 1) (layer "B.Cu") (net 12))
 (segment (start 192.6 94.12) (end 192.6 89.3) (width 1) (layer "B.Cu") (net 19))
 (segment (start 192.6 89.3) (end 194.12 87.78) (width 1) (layer "B.Cu") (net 19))
 (segment (start 194.12 87.78) (end 195.9 87.78) (width 1) (layer "B.Cu") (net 19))
 (segment (start 195.6 82.7) (end 192 79.1) (width 1) (layer "B.Cu") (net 16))
 (segment (start 181.7 68.7) (end 184.3 66.1) (width 1) (layer "B.Cu") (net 16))
 (segment (start 195.9 82.7) (end 195.6 82.7) (width 1) (layer "B.Cu") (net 16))
 (segment (start 201.5 66.1) (end 210.9 75.5) (width 1) (layer "B.Cu") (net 16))
 (segment (start 181.7 74.7) (end 181.7 68.7) (width 1) (layer "B.Cu") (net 16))
 (segment (start 192 79.1) (end 186.1 79.1) (width 1) (layer "B.Cu") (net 16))
 (segment (start 210.9 75.5) (end 210.9 80.22) (width 1) (layer "B.Cu") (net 16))
 (segment (start 210.9 80.22) (end 211.2 80.52) (width 1) (layer "B.Cu") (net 16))
 (segment (start 184.3 66.1) (end 201.5 66.1) (width 1) (layer "B.Cu") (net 16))
 (segment (start 186.1 79.1) (end 181.7 74.7) (width 1) (layer "B.Cu") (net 16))
 (segment (start 208 90.68) (end 211.2 90.68) (width 1) (layer "B.Cu") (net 18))
 (segment (start 207.48 90.68) (end 208 90.68) (width 1) (layer "B.Cu") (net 18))
 (segment (start 204.58 87.78) (end 207.48 90.68) (width 1) (layer "B.Cu") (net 18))
 (segment (start 203.52 87.78) (end 204.58 87.78) (width 1) (layer "B.Cu") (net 18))
 (segment (start 203.1 93.62) (end 203.1 90.74) (width 1) (layer "B.Cu") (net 3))
 (segment (start 203.1 90.74) (end 203.52 90.32) (width 1) (layer "B.Cu") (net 3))
 (segment (start 208 80.52) (end 208 84.9) (width 1) (layer "B.Cu") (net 10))
 (segment (start 209.54 85.24) (end 207.66 85.24) (width 1) (layer "B.Cu") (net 10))
 (segment (start 208 84.9) (end 207.66 85.24) (width 1) (layer "B.Cu") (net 10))
 (segment (start 214.4 90.1) (end 209.54 85.24) (width 1) (layer "B.Cu") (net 10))
 (segment (start 214.4 90.68) (end 214.4 90.1) (width 1) (layer "B.Cu") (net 10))
 (segment (start 207.66 85.24) (end 203.52 85.24) (width 1) (layer "B.Cu") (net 10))
 (segment (start 189.4 87.22) (end 189.4 85.64) (width 1) (layer "B.Cu") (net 14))
 (segment (start 189.4 85.64) (end 190.7 84.34) (width 1) (layer "B.Cu") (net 14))
 (segment (start 185.9 90.3) (end 186.32 90.3) (width 1) (layer "B.Cu") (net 14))
 (segment (start 186.32 90.3) (end 189.4 87.22) (width 1) (layer "B.Cu") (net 14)))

